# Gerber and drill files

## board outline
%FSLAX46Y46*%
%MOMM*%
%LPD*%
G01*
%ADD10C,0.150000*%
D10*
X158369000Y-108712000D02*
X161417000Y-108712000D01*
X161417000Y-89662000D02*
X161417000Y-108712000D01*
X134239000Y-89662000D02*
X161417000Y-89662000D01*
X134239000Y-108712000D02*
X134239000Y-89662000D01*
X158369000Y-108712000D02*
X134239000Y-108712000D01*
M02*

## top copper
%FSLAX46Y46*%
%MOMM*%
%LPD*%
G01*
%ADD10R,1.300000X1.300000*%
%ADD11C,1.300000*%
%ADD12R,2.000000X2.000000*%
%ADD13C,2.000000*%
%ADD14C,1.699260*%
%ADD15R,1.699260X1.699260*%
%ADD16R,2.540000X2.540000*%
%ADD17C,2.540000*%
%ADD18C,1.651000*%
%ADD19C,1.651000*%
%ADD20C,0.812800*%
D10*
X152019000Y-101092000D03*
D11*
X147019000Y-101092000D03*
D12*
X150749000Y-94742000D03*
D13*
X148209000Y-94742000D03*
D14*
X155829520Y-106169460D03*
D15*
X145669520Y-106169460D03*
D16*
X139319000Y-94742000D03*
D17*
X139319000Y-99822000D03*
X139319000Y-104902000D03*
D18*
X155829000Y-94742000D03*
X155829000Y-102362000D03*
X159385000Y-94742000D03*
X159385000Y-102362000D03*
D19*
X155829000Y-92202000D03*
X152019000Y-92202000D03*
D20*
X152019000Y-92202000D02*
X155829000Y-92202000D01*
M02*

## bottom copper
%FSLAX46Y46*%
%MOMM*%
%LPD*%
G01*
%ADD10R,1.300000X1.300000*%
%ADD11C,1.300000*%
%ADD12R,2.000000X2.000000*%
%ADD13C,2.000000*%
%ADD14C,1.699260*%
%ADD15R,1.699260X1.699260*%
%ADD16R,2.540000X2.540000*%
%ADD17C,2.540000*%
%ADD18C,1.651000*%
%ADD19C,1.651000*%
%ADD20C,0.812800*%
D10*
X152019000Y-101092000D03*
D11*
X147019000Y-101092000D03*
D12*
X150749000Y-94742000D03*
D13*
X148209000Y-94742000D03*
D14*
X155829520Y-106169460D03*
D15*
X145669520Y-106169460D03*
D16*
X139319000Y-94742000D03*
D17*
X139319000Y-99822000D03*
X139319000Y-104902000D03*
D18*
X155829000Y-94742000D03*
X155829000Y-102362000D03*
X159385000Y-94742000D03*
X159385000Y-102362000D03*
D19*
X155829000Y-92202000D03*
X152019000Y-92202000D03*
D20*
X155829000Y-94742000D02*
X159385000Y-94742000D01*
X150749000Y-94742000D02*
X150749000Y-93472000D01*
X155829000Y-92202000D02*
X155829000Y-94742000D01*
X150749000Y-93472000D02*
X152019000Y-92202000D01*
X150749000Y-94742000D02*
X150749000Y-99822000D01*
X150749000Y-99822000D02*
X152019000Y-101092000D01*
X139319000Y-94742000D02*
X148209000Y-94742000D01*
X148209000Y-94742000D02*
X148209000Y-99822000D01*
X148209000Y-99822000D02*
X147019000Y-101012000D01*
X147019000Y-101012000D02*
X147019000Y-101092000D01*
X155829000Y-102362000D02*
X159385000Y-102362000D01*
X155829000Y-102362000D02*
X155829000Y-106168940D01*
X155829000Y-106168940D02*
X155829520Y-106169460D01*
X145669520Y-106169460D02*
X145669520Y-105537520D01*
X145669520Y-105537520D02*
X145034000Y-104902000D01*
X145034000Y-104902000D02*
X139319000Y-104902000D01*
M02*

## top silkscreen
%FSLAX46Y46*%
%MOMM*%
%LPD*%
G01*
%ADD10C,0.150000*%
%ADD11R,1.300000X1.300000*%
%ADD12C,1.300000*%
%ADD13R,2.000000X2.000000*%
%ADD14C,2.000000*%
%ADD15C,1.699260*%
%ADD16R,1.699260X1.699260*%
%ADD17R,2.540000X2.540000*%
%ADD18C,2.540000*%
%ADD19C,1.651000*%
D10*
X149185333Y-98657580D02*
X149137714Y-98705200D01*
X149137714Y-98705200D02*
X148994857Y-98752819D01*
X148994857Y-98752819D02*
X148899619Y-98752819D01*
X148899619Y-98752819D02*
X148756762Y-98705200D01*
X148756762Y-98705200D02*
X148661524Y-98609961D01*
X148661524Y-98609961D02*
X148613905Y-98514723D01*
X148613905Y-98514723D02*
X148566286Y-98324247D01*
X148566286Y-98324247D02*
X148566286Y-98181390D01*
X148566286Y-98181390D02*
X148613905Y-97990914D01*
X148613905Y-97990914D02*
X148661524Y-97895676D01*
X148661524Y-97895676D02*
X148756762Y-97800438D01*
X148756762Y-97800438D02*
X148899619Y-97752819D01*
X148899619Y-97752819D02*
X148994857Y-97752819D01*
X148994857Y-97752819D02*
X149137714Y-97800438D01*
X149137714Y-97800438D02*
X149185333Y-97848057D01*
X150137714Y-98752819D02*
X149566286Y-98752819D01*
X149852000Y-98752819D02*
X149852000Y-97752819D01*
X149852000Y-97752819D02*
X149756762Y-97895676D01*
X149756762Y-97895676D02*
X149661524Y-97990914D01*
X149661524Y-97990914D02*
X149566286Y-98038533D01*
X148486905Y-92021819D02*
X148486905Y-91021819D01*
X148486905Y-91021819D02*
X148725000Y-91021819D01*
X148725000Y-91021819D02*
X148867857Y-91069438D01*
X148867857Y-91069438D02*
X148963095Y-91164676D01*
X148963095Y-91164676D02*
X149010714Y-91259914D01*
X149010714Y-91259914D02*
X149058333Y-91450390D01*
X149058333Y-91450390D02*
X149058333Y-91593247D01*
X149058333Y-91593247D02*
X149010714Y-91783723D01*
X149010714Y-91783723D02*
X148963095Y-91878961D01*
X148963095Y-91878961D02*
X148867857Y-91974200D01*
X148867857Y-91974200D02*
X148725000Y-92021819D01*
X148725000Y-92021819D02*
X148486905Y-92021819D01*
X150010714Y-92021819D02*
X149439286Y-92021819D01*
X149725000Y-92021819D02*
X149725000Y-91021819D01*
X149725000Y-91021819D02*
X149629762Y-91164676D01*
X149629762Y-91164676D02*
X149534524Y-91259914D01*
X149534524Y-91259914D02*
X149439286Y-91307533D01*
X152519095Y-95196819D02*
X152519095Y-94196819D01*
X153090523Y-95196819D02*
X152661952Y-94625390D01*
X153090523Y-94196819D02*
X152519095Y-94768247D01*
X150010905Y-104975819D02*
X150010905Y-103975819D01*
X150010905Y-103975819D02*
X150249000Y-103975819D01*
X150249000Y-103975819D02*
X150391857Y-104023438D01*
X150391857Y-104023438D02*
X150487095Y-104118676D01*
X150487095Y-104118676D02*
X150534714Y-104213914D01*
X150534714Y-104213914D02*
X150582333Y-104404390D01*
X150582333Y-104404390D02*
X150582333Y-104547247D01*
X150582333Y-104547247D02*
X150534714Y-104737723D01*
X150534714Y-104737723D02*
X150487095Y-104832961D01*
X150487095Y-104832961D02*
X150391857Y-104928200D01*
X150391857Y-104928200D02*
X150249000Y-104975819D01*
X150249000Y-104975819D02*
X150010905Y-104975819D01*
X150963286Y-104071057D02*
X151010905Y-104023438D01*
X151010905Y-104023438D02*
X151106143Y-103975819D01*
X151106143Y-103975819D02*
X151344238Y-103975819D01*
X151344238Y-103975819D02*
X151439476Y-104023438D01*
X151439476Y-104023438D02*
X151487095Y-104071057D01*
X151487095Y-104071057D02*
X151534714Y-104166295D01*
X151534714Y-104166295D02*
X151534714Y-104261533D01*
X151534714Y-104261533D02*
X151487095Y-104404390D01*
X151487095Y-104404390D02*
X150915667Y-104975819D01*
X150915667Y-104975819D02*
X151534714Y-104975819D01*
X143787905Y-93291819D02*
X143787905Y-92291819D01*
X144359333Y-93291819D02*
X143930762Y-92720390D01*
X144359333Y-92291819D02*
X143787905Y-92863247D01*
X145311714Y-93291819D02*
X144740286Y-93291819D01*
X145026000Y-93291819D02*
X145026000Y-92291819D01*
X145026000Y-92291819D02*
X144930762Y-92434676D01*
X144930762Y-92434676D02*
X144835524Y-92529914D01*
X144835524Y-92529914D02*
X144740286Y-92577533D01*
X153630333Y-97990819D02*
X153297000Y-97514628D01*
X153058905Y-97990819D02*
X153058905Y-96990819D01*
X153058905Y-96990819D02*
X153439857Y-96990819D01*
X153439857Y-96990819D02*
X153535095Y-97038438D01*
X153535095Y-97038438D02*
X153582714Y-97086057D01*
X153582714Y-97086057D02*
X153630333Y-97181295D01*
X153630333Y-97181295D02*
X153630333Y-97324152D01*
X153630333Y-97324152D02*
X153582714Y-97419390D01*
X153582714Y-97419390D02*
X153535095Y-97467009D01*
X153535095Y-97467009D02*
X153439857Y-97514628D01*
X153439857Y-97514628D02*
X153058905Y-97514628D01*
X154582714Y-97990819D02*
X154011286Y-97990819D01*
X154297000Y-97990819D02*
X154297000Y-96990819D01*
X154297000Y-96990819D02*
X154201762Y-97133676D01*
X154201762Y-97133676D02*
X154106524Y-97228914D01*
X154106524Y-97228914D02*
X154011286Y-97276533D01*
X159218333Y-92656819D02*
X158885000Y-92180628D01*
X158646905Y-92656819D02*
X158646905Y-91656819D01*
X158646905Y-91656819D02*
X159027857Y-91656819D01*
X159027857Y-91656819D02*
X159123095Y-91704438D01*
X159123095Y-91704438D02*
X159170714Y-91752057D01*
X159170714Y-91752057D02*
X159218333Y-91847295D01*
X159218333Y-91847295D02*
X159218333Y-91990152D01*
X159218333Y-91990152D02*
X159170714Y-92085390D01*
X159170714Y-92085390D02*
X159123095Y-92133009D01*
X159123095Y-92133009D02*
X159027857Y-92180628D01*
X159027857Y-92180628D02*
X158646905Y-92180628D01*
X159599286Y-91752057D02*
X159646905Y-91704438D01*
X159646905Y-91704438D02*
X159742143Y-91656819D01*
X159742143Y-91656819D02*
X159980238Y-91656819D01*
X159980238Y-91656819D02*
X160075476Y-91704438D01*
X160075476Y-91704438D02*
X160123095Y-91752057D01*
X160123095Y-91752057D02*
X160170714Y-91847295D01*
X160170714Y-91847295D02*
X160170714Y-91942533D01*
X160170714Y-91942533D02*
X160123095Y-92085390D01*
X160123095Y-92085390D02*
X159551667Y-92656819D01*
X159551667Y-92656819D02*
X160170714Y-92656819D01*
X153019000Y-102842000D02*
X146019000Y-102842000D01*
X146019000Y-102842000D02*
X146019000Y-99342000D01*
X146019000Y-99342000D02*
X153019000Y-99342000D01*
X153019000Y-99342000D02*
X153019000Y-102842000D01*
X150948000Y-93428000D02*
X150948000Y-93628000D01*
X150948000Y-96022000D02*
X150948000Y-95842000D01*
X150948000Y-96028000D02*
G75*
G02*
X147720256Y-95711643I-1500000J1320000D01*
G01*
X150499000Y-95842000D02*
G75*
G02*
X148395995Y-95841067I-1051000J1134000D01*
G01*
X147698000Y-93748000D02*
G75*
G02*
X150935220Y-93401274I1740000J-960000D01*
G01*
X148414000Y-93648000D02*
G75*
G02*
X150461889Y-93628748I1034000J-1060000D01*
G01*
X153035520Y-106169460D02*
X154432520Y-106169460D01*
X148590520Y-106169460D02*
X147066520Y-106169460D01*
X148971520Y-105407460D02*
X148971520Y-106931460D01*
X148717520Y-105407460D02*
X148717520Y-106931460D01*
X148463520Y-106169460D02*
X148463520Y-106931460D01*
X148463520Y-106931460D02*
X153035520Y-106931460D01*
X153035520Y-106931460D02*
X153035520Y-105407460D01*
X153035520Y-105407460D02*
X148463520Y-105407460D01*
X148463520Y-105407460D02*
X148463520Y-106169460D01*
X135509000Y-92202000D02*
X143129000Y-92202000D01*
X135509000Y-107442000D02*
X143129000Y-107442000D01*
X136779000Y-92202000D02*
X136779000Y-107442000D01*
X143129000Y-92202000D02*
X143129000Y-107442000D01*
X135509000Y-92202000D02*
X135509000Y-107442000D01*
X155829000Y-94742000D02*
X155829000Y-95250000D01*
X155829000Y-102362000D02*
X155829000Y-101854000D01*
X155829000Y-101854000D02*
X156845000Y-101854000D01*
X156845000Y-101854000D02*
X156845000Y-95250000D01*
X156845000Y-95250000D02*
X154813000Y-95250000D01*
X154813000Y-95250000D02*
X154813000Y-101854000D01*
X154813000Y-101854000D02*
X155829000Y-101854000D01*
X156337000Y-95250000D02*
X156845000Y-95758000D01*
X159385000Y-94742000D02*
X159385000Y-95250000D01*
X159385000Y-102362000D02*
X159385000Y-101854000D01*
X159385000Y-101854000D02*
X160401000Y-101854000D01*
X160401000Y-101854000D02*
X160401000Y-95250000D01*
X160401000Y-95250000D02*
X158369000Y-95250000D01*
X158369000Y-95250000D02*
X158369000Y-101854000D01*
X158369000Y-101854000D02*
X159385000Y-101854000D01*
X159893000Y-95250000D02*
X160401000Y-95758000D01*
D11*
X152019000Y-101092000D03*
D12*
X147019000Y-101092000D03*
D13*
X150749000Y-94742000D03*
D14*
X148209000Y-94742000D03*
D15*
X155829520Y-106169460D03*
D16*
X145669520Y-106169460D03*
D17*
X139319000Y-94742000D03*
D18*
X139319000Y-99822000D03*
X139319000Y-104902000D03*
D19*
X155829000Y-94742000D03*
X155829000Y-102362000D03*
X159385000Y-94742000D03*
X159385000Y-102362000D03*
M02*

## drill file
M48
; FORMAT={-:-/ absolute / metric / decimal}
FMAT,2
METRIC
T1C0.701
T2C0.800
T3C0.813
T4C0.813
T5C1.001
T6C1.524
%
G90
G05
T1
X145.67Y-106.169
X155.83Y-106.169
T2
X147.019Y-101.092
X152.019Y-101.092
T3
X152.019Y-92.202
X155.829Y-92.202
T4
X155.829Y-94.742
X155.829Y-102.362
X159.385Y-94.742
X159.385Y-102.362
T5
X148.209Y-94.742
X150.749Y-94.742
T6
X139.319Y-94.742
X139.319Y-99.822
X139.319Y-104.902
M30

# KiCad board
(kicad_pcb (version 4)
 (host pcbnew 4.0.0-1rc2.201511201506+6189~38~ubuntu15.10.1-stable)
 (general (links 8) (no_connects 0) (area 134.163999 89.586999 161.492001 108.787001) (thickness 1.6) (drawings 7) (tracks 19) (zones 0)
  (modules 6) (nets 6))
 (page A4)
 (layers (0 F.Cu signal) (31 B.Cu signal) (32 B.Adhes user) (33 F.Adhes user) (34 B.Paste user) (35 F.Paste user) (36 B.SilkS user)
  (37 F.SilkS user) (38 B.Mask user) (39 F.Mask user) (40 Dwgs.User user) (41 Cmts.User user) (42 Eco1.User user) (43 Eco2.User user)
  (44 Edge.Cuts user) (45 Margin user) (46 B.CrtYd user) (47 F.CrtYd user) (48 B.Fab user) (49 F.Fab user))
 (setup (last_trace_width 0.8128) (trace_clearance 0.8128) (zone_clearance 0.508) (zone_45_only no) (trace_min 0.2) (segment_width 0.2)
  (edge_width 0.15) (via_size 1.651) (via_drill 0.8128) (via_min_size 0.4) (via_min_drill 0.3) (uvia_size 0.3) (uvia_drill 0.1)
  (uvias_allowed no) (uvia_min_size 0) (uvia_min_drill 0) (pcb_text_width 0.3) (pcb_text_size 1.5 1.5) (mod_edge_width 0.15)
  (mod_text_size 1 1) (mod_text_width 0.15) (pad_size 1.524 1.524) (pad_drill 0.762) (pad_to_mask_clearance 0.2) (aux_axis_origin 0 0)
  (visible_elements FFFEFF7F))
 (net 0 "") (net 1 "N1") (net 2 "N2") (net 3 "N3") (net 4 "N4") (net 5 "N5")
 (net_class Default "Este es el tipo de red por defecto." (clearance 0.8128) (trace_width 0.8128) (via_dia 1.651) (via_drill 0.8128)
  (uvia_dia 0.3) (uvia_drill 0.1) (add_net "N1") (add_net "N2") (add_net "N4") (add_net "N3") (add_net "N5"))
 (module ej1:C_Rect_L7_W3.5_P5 (layer F.Cu) (at 152.019 101.092 180)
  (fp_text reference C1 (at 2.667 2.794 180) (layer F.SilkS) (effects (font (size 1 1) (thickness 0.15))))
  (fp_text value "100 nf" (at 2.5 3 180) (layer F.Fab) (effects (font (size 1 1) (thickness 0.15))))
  (fp_line (start -1 -1.75) (end 6 -1.75) (layer F.SilkS) (width 0.15))
  (fp_line (start 6 -1.75) (end 6 1.75) (layer F.SilkS) (width 0.15))
  (fp_line (start 6 1.75) (end -1 1.75) (layer F.SilkS) (width 0.15))
  (fp_line (start -1 1.75) (end -1 -1.75) (layer F.SilkS) (width 0.15))
  (pad 1 thru_hole rect (at 0 0 180) (size 1.3 1.3) (drill 0.8) (layers *.Cu *.Mask F.SilkS) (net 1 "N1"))
  (pad 2 thru_hole circle (at 5 0 180) (size 1.3 1.3) (drill 0.8) (layers *.Cu *.Mask F.SilkS) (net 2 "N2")))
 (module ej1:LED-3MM (layer F.Cu) (at 150.749 94.742 180)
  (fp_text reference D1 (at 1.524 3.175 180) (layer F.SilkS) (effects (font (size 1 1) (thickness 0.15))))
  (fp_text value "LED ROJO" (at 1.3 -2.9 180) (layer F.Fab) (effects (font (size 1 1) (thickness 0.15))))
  (fp_line (start -0.199 1.314) (end -0.199 1.114) (layer F.SilkS) (width 0.15))
  (fp_line (start -0.199 -1.28) (end -0.199 -1.1) (layer F.SilkS) (width 0.15))
  (fp_arc (start 1.301 0.034) (end -0.199 -1.286) (angle 108.5) (layer F.SilkS) (width 0.15))
  (fp_arc (start 1.301 0.034) (end 0.25 -1.1) (angle 85.7) (layer F.SilkS) (width 0.15))
  (fp_arc (start 1.311 0.034) (end 3.051 0.994) (angle 110) (layer F.SilkS) (width 0.15))
  (fp_arc (start 1.301 0.034) (end 2.335 1.094) (angle 87.5) (layer F.SilkS) (width 0.15))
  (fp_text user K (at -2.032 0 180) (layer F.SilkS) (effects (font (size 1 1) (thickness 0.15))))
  (pad 1 thru_hole rect (at 0 0 270) (size 2 2) (drill 1.00076) (layers *.Cu *.Mask F.SilkS) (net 1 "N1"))
  (pad 2 thru_hole circle (at 2.54 0 180) (size 2 2) (drill 1.00076) (layers *.Cu *.Mask F.SilkS) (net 2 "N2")))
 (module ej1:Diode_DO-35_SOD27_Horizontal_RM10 (layer F.Cu) (at 145.669 106.172)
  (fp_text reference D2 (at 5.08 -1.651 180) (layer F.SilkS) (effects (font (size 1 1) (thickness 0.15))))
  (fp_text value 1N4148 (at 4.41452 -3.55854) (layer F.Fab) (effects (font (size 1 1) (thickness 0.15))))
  (fp_line (start 7.36652 -0.00254) (end 8.76352 -0.00254) (layer F.SilkS) (width 0.15))
  (fp_line (start 2.92152 -0.00254) (end 1.39752 -0.00254) (layer F.SilkS) (width 0.15))
  (fp_line (start 3.30252 -0.76454) (end 3.30252 0.75946) (layer F.SilkS) (width 0.15))
  (fp_line (start 3.04852 -0.76454) (end 3.04852 0.75946) (layer F.SilkS) (width 0.15))
  (fp_line (start 2.79452 -0.00254) (end 2.79452 0.75946) (layer F.SilkS) (width 0.15))
  (fp_line (start 2.79452 0.75946) (end 7.36652 0.75946) (layer F.SilkS) (width 0.15))
  (fp_line (start 7.36652 0.75946) (end 7.36652 -0.76454) (layer F.SilkS) (width 0.15))
  (fp_line (start 7.36652 -0.76454) (end 2.79452 -0.76454) (layer F.SilkS) (width 0.15))
  (fp_line (start 2.79452 -0.76454) (end 2.79452 -0.00254) (layer F.SilkS) (width 0.15))
  (pad 2 thru_hole circle (at 10.16052 -0.00254 180) (size 1.69926 1.69926) (drill 0.70104) (layers *.Cu *.Mask F.SilkS) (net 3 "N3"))
  (pad 1 thru_hole rect (at 0.00052 -0.00254 180) (size 1.69926 1.69926) (drill 0.70104) (layers *.Cu *.Mask F.SilkS) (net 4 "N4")))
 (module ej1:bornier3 (layer F.Cu) (at 139.319 99.822 270)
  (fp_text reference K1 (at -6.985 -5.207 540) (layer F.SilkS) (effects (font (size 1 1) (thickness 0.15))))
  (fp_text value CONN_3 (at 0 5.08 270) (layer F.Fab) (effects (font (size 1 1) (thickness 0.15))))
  (fp_line (start -7.62 3.81) (end -7.62 -3.81) (layer F.SilkS) (width 0.15))
  (fp_line (start 7.62 3.81) (end 7.62 -3.81) (layer F.SilkS) (width 0.15))
  (fp_line (start -7.62 2.54) (end 7.62 2.54) (layer F.SilkS) (width 0.15))
  (fp_line (start -7.62 -3.81) (end 7.62 -3.81) (layer F.SilkS) (width 0.15))
  (fp_line (start -7.62 3.81) (end 7.62 3.81) (layer F.SilkS) (width 0.15))
  (pad 1 thru_hole rect (at -5.08 0 270) (size 2.54 2.54) (drill 1.524) (layers *.Cu *.Mask F.SilkS) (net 2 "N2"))
  (pad 2 thru_hole circle (at 0 0 270) (size 2.54 2.54) (drill 1.524) (layers *.Cu *.Mask F.SilkS) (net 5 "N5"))
  (pad 3 thru_hole circle (at 5.08 0 270) (size 2.54 2.54) (drill 1.524) (layers *.Cu *.Mask F.SilkS) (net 4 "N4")))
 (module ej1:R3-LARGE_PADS (layer F.Cu) (at 155.829 98.552 270)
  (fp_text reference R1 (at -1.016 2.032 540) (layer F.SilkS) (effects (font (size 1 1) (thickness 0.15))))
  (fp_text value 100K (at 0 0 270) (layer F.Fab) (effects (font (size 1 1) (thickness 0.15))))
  (fp_line (start -3.81 0) (end -3.302 0) (layer F.SilkS) (width 0.15))
  (fp_line (start 3.81 0) (end 3.302 0) (layer F.SilkS) (width 0.15))
  (fp_line (start 3.302 0) (end 3.302 -1.016) (layer F.SilkS) (width 0.15))
  (fp_line (start 3.302 -1.016) (end -3.302 -1.016) (layer F.SilkS) (width 0.15))
  (fp_line (start -3.302 -1.016) (end -3.302 1.016) (layer F.SilkS) (width 0.15))
  (fp_line (start -3.302 1.016) (end 3.302 1.016) (layer F.SilkS) (width 0.15))
  (fp_line (start 3.302 1.016) (end 3.302 0) (layer F.SilkS) (width 0.15))
  (fp_line (start -3.302 -0.508) (end -2.794 -1.016) (layer F.SilkS) (width 0.15))
  (pad 1 thru_hole circle (at -3.81 0 270) (size 1.651 1.651) (drill 0.8128) (layers *.Cu *.Mask F.SilkS) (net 1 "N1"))
  (pad 2 thru_hole circle (at 3.81 0 270) (size 1.651 1.651) (drill 0.8128) (layers *.Cu *.Mask F.SilkS) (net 3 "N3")))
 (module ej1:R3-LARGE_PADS (layer F.Cu) (at 159.385 98.552 270)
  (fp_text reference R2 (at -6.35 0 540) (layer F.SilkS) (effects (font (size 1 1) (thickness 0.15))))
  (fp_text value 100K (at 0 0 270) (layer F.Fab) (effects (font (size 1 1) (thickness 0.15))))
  (fp_line (start -3.81 0) (end -3.302 0) (layer F.SilkS) (width 0.15))
  (fp_line (start 3.81 0) (end 3.302 0) (layer F.SilkS) (width 0.15))
  (fp_line (start 3.302 0) (end 3.302 -1.016) (layer F.SilkS) (width 0.15))
  (fp_line (start 3.302 -1.016) (end -3.302 -1.016) (layer F.SilkS) (width 0.15))
  (fp_line (start -3.302 -1.016) (end -3.302 1.016) (layer F.SilkS) (width 0.15))
  (fp_line (start -3.302 1.016) (end 3.302 1.016) (layer F.SilkS) (width 0.15))
  (fp_line (start 3.302 1.016) (end 3.302 0) (layer F.SilkS) (width 0.15))
  (fp_line (start -3.302 -0.508) (end -2.794 -1.016) (layer F.SilkS) (width 0.15))
  (pad 1 thru_hole circle (at -3.81 0 270) (size 1.651 1.651) (drill 0.8128) (layers *.Cu *.Mask F.SilkS) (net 1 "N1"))
  (pad 2 thru_hole circle (at 3.81 0 270) (size 1.651 1.651) (drill 0.8128) (layers *.Cu *.Mask F.SilkS) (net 3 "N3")))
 (gr_line (start 158.369 108.712) (end 161.417 108.712) (angle 90) (layer Edge.Cuts) (width 0.15))
 (gr_line (start 161.417 89.662) (end 161.417 108.712) (angle 90) (layer Edge.Cuts) (width 0.15))
 (gr_line (start 134.239 89.662) (end 161.417 89.662) (angle 90) (layer Edge.Cuts) (width 0.15))
 (gr_line (start 134.239 108.712) (end 134.239 89.662) (angle 90) (layer Edge.Cuts) (width 0.15))
 (gr_line (start 158.369 108.712) (end 134.239 108.712) (angle 90) (layer Edge.Cuts) (width 0.15))
 (segment (start 155.829 94.742) (end 159.385 94.742) (width 0.8128) (layer B.Cu) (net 1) (status C00000))
 (segment (start 150.749 94.742) (end 150.749 93.472) (width 0.8128) (layer B.Cu) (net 1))
 (segment (start 155.829 92.202) (end 155.829 94.742) (width 0.8128) (layer B.Cu) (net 1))
 (via (at 155.829 92.202) (size 1.651) (drill 0.8128) (layers F.Cu B.Cu) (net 1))
 (segment (start 152.019 92.202) (end 155.829 92.202) (width 0.8128) (layer F.Cu) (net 1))
 (via (at 152.019 92.202) (size 1.651) (drill 0.8128) (layers F.Cu B.Cu) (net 1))
 (segment (start 150.749 93.472) (end 152.019 92.202) (width 0.8128) (layer B.Cu) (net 1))
 (segment (start 150.749 94.742) (end 150.749 99.822) (width 0.8128) (layer B.Cu) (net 1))
 (segment (start 150.749 99.822) (end 152.019 101.092) (width 0.8128) (layer B.Cu) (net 1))
 (segment (start 139.319 94.742) (end 148.209 94.742) (width 0.8128) (layer B.Cu) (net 2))
 (segment (start 148.209 94.742) (end 148.209 99.822) (width 0.8128) (layer B.Cu) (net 2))
 (segment (start 148.209 99.822) (end 147.019 101.012) (width 0.8128) (layer B.Cu) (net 2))
 (segment (start 147.019 101.012) (end 147.019 101.092) (width 0.8128) (layer B.Cu) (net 2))
 (segment (start 155.829 102.362) (end 159.385 102.362) (width 0.8128) (layer B.Cu) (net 3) (status C00000))
 (segment (start 155.829 102.362) (end 155.829 106.16894) (width 0.8128) (layer B.Cu) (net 3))
 (segment (start 155.829 106.16894) (end 155.82952 106.16946) (width 0.8128) (layer B.Cu) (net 3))
 (segment (start 145.66952 106.16946) (end 145.66952 105.53752) (width 0.8128) (layer B.Cu) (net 4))
 (segment (start 145.66952 105.53752) (end 145.034 104.902) (width 0.8128) (layer B.Cu) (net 4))
 (segment (start 145.034 104.902) (end 139.319 104.902) (width 0.8128) (layer B.Cu) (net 4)))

